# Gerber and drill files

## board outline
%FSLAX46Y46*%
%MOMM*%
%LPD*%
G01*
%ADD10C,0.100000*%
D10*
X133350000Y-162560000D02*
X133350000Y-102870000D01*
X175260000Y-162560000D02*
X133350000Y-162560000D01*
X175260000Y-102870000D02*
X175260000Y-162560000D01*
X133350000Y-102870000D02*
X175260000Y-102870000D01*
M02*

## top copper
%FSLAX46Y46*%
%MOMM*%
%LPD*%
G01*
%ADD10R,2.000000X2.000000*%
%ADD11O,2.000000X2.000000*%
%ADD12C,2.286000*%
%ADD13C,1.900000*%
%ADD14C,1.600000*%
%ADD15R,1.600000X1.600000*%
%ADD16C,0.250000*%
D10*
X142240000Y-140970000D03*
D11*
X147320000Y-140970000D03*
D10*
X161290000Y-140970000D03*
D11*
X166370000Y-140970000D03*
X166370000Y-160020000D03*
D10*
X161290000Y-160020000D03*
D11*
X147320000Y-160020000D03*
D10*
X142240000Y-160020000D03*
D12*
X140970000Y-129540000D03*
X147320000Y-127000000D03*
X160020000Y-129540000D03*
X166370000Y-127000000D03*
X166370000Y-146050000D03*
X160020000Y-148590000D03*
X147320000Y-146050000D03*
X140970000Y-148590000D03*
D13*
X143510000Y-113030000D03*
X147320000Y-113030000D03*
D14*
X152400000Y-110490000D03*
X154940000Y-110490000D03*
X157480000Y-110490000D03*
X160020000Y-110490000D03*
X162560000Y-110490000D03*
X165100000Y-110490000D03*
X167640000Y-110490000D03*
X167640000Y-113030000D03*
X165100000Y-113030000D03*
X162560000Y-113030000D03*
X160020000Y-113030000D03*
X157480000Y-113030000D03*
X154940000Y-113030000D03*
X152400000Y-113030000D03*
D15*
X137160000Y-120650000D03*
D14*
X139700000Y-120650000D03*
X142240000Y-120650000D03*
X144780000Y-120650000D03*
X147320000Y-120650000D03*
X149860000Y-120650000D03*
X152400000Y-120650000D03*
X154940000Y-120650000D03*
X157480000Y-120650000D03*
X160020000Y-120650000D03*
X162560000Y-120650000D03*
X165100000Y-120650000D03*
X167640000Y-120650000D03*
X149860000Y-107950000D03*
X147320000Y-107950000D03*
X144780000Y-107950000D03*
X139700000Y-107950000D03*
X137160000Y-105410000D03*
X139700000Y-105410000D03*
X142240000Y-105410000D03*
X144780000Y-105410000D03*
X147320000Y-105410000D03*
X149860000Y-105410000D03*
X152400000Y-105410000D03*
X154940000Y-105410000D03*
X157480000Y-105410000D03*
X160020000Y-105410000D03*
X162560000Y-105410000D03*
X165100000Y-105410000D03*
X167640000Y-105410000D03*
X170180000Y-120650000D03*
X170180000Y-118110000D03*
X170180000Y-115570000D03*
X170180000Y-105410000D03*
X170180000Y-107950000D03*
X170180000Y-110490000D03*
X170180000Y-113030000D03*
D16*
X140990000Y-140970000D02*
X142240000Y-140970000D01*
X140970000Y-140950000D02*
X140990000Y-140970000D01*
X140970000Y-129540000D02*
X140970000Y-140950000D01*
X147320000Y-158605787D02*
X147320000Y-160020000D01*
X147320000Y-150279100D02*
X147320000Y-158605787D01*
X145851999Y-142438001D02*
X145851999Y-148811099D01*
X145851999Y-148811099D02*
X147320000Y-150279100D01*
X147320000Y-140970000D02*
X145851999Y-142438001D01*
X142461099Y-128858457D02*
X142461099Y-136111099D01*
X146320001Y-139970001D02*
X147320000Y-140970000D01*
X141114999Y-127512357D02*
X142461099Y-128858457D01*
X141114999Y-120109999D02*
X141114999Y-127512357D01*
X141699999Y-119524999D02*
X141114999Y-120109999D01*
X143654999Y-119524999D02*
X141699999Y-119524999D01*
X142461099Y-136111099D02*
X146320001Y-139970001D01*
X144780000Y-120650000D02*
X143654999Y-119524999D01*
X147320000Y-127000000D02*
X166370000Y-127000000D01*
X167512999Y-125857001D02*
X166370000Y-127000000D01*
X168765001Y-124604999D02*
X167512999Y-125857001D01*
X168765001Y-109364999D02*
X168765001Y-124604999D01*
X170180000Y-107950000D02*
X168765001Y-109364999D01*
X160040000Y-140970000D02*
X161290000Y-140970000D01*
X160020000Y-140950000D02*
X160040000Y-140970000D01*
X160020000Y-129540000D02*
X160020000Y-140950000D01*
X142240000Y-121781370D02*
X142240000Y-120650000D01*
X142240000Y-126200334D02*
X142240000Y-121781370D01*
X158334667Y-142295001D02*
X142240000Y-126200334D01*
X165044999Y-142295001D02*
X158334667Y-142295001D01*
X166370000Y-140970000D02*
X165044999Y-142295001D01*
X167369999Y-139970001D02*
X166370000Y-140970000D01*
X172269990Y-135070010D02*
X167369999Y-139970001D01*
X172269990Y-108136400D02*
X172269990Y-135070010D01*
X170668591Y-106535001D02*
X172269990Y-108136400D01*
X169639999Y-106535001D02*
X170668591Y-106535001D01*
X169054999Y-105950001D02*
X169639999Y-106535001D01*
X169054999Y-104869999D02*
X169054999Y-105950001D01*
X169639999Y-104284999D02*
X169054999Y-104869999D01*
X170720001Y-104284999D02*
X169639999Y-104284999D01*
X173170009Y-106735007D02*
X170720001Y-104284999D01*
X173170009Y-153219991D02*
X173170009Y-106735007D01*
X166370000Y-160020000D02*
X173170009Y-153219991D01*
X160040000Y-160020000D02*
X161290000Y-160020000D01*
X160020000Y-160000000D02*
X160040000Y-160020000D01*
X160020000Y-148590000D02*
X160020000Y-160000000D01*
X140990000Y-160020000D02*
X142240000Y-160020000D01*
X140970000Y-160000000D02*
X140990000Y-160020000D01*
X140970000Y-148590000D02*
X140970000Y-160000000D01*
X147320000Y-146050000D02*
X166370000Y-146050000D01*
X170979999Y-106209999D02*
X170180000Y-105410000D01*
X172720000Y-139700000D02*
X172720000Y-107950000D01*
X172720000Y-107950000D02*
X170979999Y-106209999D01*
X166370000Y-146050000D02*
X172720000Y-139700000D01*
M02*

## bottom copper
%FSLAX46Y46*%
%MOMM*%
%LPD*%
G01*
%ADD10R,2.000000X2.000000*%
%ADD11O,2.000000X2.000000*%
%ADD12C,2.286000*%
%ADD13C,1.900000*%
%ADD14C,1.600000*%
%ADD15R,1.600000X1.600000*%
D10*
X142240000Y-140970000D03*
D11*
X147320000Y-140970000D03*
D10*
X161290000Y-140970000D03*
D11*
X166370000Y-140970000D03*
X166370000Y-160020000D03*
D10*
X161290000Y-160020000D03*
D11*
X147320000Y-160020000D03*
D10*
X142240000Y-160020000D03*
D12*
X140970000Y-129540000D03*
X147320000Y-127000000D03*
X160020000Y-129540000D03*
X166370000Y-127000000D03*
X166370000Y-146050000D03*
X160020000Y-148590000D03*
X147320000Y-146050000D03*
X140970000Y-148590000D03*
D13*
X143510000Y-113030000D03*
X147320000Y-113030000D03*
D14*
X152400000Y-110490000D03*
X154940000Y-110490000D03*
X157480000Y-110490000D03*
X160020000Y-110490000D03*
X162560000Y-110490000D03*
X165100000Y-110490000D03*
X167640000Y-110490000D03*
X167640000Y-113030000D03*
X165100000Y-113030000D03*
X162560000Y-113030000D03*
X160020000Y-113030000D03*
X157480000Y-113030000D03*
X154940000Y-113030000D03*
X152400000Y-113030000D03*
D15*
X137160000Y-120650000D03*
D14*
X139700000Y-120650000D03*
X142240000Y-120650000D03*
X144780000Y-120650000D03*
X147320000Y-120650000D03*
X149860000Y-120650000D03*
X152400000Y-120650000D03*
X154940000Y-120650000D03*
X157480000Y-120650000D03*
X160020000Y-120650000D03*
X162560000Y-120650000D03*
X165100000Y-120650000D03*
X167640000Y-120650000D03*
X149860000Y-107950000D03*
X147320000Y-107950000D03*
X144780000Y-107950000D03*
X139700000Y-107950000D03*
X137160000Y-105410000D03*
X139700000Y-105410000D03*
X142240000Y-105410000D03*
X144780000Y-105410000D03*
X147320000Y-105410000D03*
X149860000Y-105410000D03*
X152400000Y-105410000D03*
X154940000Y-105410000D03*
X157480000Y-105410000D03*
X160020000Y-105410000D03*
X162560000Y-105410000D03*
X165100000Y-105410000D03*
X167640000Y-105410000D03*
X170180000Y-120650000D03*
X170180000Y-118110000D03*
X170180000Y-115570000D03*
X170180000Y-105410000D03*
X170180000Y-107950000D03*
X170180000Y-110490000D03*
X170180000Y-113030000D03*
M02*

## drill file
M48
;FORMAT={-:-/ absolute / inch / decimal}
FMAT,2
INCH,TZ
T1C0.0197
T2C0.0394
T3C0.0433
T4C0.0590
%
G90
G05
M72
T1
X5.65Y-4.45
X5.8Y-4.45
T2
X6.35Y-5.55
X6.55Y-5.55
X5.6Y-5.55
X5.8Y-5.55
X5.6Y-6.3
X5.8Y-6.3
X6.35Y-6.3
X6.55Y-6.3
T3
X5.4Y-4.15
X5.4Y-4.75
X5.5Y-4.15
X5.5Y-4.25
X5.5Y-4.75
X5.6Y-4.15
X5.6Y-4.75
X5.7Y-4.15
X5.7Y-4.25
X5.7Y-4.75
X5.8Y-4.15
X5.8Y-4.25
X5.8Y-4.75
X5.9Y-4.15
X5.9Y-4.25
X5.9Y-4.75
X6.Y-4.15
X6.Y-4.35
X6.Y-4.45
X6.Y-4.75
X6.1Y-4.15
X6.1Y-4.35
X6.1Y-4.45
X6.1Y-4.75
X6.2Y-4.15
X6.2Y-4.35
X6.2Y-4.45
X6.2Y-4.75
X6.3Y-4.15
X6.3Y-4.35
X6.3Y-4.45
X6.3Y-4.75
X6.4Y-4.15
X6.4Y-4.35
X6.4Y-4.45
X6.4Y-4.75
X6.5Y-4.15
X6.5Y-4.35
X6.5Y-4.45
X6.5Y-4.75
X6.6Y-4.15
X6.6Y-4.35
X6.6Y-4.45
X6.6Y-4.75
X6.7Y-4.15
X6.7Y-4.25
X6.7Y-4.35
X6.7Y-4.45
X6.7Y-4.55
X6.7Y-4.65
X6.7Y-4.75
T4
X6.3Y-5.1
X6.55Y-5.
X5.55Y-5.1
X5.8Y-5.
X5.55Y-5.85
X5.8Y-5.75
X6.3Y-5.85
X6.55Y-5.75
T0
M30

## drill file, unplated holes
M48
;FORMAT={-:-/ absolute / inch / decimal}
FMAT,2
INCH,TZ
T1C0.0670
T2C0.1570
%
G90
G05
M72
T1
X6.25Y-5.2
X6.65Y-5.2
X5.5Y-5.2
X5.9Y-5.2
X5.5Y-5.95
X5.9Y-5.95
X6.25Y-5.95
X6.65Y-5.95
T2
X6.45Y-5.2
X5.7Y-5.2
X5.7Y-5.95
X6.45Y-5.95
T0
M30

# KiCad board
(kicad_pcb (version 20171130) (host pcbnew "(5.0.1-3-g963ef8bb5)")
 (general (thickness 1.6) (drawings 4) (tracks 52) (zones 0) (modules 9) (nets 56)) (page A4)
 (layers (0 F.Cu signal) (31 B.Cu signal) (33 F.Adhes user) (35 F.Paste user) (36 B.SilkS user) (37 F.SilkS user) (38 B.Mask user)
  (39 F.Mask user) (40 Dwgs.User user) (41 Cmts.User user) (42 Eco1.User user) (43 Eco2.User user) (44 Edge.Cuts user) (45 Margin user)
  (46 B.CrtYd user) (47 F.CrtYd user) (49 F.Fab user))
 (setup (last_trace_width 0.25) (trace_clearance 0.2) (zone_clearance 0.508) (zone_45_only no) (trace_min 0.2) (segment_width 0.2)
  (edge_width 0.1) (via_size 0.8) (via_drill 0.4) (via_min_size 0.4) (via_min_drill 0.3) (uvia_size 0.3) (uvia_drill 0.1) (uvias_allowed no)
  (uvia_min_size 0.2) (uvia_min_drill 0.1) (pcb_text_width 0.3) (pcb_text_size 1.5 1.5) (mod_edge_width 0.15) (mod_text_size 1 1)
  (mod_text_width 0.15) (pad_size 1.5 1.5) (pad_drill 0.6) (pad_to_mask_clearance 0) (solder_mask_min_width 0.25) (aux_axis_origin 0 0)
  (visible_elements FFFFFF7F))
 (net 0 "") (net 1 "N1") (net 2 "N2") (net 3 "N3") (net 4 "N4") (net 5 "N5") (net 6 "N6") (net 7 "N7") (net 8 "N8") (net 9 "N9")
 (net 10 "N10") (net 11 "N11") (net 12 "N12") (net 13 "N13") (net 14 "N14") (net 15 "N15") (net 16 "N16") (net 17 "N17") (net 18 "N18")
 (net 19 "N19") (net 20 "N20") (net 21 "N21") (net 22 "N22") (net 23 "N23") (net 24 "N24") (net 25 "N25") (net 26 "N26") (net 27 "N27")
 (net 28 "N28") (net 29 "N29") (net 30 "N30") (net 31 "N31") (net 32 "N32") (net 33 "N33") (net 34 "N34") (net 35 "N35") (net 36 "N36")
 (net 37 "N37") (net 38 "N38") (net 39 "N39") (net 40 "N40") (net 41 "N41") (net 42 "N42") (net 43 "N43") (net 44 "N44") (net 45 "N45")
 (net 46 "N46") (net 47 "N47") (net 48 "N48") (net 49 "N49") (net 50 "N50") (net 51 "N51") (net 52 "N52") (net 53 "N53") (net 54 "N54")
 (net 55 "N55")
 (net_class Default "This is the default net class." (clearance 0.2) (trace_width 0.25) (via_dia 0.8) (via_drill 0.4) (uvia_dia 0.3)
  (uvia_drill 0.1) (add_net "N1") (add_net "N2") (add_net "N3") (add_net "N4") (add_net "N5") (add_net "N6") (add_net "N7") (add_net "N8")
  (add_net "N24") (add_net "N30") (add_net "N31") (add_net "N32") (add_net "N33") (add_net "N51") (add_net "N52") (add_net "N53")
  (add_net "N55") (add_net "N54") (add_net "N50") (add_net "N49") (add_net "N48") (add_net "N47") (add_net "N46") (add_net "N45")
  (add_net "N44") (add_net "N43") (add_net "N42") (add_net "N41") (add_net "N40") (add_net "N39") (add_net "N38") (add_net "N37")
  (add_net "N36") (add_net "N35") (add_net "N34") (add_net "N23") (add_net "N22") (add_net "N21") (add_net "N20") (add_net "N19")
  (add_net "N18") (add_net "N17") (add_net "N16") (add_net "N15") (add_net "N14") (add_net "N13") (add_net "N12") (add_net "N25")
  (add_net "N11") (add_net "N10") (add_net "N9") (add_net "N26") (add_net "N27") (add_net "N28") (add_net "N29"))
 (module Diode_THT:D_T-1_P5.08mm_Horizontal (layer F.Cu) (at 142.24 140.97)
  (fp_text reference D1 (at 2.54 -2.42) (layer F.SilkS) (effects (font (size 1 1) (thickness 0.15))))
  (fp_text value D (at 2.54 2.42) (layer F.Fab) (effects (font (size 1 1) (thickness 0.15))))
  (pad 1 thru_hole rect (at 0 0) (size 2 2) (drill 1) (layers *.Cu *.Mask) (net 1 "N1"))
  (pad 2 thru_hole oval (at 5.08 0) (size 2 2) (drill 1) (layers *.Cu *.Mask) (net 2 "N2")))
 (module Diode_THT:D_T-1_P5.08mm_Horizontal (layer F.Cu) (at 161.29 140.97)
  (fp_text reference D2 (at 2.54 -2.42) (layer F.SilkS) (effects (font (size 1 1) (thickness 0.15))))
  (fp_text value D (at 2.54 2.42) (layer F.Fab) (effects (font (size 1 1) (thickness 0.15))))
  (pad 1 thru_hole rect (at 0 0) (size 2 2) (drill 1) (layers *.Cu *.Mask) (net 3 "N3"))
  (pad 2 thru_hole oval (at 5.08 0) (size 2 2) (drill 1) (layers *.Cu *.Mask) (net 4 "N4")))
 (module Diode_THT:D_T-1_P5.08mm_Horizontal (layer F.Cu) (at 161.29 160.02)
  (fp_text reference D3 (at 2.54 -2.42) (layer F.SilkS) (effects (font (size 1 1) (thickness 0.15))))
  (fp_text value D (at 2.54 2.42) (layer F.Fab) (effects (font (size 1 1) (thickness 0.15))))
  (pad 2 thru_hole oval (at 5.08 0) (size 2 2) (drill 1) (layers *.Cu *.Mask) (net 4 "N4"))
  (pad 1 thru_hole rect (at 0 0) (size 2 2) (drill 1) (layers *.Cu *.Mask) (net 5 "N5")))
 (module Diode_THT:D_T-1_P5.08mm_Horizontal (layer F.Cu) (at 142.24 160.02)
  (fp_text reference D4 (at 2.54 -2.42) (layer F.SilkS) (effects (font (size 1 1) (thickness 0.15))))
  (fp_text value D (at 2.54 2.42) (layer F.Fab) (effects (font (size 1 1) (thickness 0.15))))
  (pad 2 thru_hole oval (at 5.08 0) (size 2 2) (drill 1) (layers *.Cu *.Mask) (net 2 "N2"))
  (pad 1 thru_hole rect (at 0 0) (size 2 2) (drill 1) (layers *.Cu *.Mask) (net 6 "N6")))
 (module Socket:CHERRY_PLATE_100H (layer F.Cu) (at 144.78 132.08)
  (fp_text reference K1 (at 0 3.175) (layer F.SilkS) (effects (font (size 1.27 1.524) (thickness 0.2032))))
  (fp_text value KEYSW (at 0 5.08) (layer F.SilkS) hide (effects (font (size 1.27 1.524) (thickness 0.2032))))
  (pad HOLE np_thru_hole circle (at 5.08 0) (size 1.7018 1.7018) (drill 1.7018) (layers *.Cu))
  (pad HOLE np_thru_hole circle (at -5.08 0) (size 1.7018 1.7018) (drill 1.7018) (layers *.Cu))
  (pad HOLE np_thru_hole circle (at 0 0) (size 3.9878 3.9878) (drill 3.9878) (layers *.Cu))
  (pad 2 thru_hole circle (at -3.81 -2.54) (size 2.286 2.286) (drill 1.4986) (layers *.Cu *.SilkS *.Mask) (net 1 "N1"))
  (pad 1 thru_hole circle (at 2.54 -5.08) (size 2.286 2.286) (drill 1.4986) (layers *.Cu *.SilkS *.Mask) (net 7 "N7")))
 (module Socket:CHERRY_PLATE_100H (layer F.Cu) (at 163.83 132.08)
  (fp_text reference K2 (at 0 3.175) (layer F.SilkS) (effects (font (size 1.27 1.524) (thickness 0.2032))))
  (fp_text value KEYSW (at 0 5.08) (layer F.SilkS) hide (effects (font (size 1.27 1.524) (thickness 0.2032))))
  (pad HOLE np_thru_hole circle (at 5.08 0) (size 1.7018 1.7018) (drill 1.7018) (layers *.Cu))
  (pad HOLE np_thru_hole circle (at -5.08 0) (size 1.7018 1.7018) (drill 1.7018) (layers *.Cu))
  (pad HOLE np_thru_hole circle (at 0 0) (size 3.9878 3.9878) (drill 3.9878) (layers *.Cu))
  (pad 2 thru_hole circle (at -3.81 -2.54) (size 2.286 2.286) (drill 1.4986) (layers *.Cu *.SilkS *.Mask) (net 3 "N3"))
  (pad 1 thru_hole circle (at 2.54 -5.08) (size 2.286 2.286) (drill 1.4986) (layers *.Cu *.SilkS *.Mask) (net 7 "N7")))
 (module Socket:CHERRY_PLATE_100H (layer F.Cu) (at 163.83 151.13)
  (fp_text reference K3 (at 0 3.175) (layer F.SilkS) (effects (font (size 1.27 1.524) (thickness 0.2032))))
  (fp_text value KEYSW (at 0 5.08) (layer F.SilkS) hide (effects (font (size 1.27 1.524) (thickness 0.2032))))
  (pad 1 thru_hole circle (at 2.54 -5.08) (size 2.286 2.286) (drill 1.4986) (layers *.Cu *.SilkS *.Mask) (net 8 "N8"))
  (pad 2 thru_hole circle (at -3.81 -2.54) (size 2.286 2.286) (drill 1.4986) (layers *.Cu *.SilkS *.Mask) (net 5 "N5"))
  (pad HOLE np_thru_hole circle (at 0 0) (size 3.9878 3.9878) (drill 3.9878) (layers *.Cu))
  (pad HOLE np_thru_hole circle (at -5.08 0) (size 1.7018 1.7018) (drill 1.7018) (layers *.Cu))
  (pad HOLE np_thru_hole circle (at 5.08 0) (size 1.7018 1.7018) (drill 1.7018) (layers *.Cu)))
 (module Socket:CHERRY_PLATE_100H (layer F.Cu) (at 144.78 151.13)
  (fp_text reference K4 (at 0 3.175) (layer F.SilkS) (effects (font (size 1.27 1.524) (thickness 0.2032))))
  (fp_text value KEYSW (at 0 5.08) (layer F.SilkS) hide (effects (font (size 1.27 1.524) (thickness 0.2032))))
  (pad 1 thru_hole circle (at 2.54 -5.08) (size 2.286 2.286) (drill 1.4986) (layers *.Cu *.SilkS *.Mask) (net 8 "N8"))
  (pad 2 thru_hole circle (at -3.81 -2.54) (size 2.286 2.286) (drill 1.4986) (layers *.Cu *.SilkS *.Mask) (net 6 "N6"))
  (pad HOLE np_thru_hole circle (at 0 0) (size 3.9878 3.9878) (drill 3.9878) (layers *.Cu))
  (pad HOLE np_thru_hole circle (at -5.08 0) (size 1.7018 1.7018) (drill 1.7018) (layers *.Cu))
  (pad HOLE np_thru_hole circle (at 5.08 0) (size 1.7018 1.7018) (drill 1.7018) (layers *.Cu)))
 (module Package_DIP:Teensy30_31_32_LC (layer F.Cu) (at 153.67 113.03)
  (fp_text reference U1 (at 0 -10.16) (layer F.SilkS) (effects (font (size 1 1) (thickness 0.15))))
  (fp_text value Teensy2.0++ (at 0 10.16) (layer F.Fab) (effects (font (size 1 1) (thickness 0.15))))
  (pad 52 thru_hole circle (at -10.16 0) (size 1.9 1.9) (drill 0.5) (layers *.Cu *.Mask F.SilkS) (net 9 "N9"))
  (pad 52 thru_hole circle (at -6.35 0) (size 1.9 1.9) (drill 0.5) (layers *.Cu *.Mask F.SilkS) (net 9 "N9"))
  (pad 51 thru_hole circle (at -1.27 -2.54) (size 1.6 1.6) (drill 1.1) (layers *.Cu *.Mask) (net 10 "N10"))
  (pad 50 thru_hole circle (at 1.27 -2.54) (size 1.6 1.6) (drill 1.1) (layers *.Cu *.Mask) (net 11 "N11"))
  (pad 49 thru_hole circle (at 3.81 -2.54) (size 1.6 1.6) (drill 1.1) (layers *.Cu *.Mask) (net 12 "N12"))
  (pad 48 thru_hole circle (at 6.35 -2.54) (size 1.6 1.6) (drill 1.1) (layers *.Cu *.Mask) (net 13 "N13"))
  (pad 47 thru_hole circle (at 8.89 -2.54) (size 1.6 1.6) (drill 1.1) (layers *.Cu *.Mask) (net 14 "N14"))
  (pad 46 thru_hole circle (at 11.43 -2.54) (size 1.6 1.6) (drill 1.1) (layers *.Cu *.Mask) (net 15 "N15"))
  (pad 45 thru_hole circle (at 13.97 -2.54) (size 1.6 1.6) (drill 1.1) (layers *.Cu *.Mask) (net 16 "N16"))
  (pad 44 thru_hole circle (at 13.97 0) (size 1.6 1.6) (drill 1.1) (layers *.Cu *.Mask) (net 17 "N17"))
  (pad 43 thru_hole circle (at 11.43 0) (size 1.6 1.6) (drill 1.1) (layers *.Cu *.Mask) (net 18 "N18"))
  (pad 42 thru_hole circle (at 8.89 0) (size 1.6 1.6) (drill 1.1) (layers *.Cu *.Mask) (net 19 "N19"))
  (pad 41 thru_hole circle (at 6.35 0) (size 1.6 1.6) (drill 1.1) (layers *.Cu *.Mask) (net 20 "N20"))
  (pad 40 thru_hole circle (at 3.81 0) (size 1.6 1.6) (drill 1.1) (layers *.Cu *.Mask) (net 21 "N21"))
  (pad 39 thru_hole circle (at 1.27 0) (size 1.6 1.6) (drill 1.1) (layers *.Cu *.Mask) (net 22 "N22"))
  (pad 38 thru_hole circle (at -1.27 0) (size 1.6 1.6) (drill 1.1) (layers *.Cu *.Mask) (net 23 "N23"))
  (pad 1 thru_hole rect (at -16.51 7.62) (size 1.6 1.6) (drill 1.1) (layers *.Cu *.Mask F.SilkS) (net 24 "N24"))
  (pad 2 thru_hole circle (at -13.97 7.62) (size 1.6 1.6) (drill 1.1) (layers *.Cu *.Mask F.SilkS))
  (pad 3 thru_hole circle (at -11.43 7.62) (size 1.6 1.6) (drill 1.1) (layers *.Cu *.Mask F.SilkS) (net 4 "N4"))
  (pad 4 thru_hole circle (at -8.89 7.62) (size 1.6 1.6) (drill 1.1) (layers *.Cu *.Mask F.SilkS) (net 2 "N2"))
  (pad 5 thru_hole circle (at -6.35 7.62) (size 1.6 1.6) (drill 1.1) (layers *.Cu *.Mask F.SilkS) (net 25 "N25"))
  (pad 6 thru_hole circle (at -3.81 7.62) (size 1.6 1.6) (drill 1.1) (layers *.Cu *.Mask F.SilkS) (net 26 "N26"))
  (pad 7 thru_hole circle (at -1.27 7.62) (size 1.6 1.6) (drill 1.1) (layers *.Cu *.Mask F.SilkS) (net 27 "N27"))
  (pad 8 thru_hole circle (at 1.27 7.62) (size 1.6 1.6) (drill 1.1) (layers *.Cu *.Mask F.SilkS) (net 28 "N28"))
  (pad 9 thru_hole circle (at 3.81 7.62) (size 1.6 1.6) (drill 1.1) (layers *.Cu *.Mask F.SilkS) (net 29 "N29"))
  (pad 10 thru_hole circle (at 6.35 7.62) (size 1.6 1.6) (drill 1.1) (layers *.Cu *.Mask F.SilkS) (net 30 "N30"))
  (pad 11 thru_hole circle (at 8.89 7.62) (size 1.6 1.6) (drill 1.1) (layers *.Cu *.Mask F.SilkS) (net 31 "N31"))
  (pad 12 thru_hole circle (at 11.43 7.62) (size 1.6 1.6) (drill 1.1) (layers *.Cu *.Mask F.SilkS) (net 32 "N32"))
  (pad 13 thru_hole circle (at 13.97 7.62) (size 1.6 1.6) (drill 1.1) (layers *.Cu *.Mask F.SilkS) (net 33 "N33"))
  (pad 37 thru_hole circle (at -3.81 -5.08) (size 1.6 1.6) (drill 1.1) (layers *.Cu *.Mask F.SilkS) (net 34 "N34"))
  (pad 36 thru_hole circle (at -6.35 -5.08) (size 1.6 1.6) (drill 1.1) (layers *.Cu *.Mask F.SilkS) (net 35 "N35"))
  (pad 35 thru_hole circle (at -8.89 -5.08) (size 1.6 1.6) (drill 1.1) (layers *.Cu *.Mask F.SilkS) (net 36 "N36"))
  (pad 34 thru_hole circle (at -13.97 -5.08) (size 1.6 1.6) (drill 1.1) (layers *.Cu *.Mask F.SilkS) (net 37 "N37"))
  (pad 33 thru_hole circle (at -16.51 -7.62) (size 1.6 1.6) (drill 1.1) (layers *.Cu *.Mask F.SilkS) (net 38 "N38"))
  (pad 32 thru_hole circle (at -13.97 -7.62) (size 1.6 1.6) (drill 1.1) (layers *.Cu *.Mask F.SilkS) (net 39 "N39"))
  (pad 31 thru_hole circle (at -11.43 -7.62) (size 1.6 1.6) (drill 1.1) (layers *.Cu *.Mask F.SilkS) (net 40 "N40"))
  (pad 30 thru_hole circle (at -8.89 -7.62) (size 1.6 1.6) (drill 1.1) (layers *.Cu *.Mask F.SilkS) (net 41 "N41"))
  (pad 29 thru_hole circle (at -6.35 -7.62) (size 1.6 1.6) (drill 1.1) (layers *.Cu *.Mask F.SilkS) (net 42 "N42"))
  (pad 28 thru_hole circle (at -3.81 -7.62) (size 1.6 1.6) (drill 1.1) (layers *.Cu *.Mask F.SilkS) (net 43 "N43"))
  (pad 27 thru_hole circle (at -1.27 -7.62) (size 1.6 1.6) (drill 1.1) (layers *.Cu *.Mask F.SilkS) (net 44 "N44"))
  (pad 26 thru_hole circle (at 1.27 -7.62) (size 1.6 1.6) (drill 1.1) (layers *.Cu *.Mask F.SilkS) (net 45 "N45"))
  (pad 25 thru_hole circle (at 3.81 -7.62) (size 1.6 1.6) (drill 1.1) (layers *.Cu *.Mask F.SilkS) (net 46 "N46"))
  (pad 24 thru_hole circle (at 6.35 -7.62) (size 1.6 1.6) (drill 1.1) (layers *.Cu *.Mask F.SilkS) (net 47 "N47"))
  (pad 23 thru_hole circle (at 8.89 -7.62) (size 1.6 1.6) (drill 1.1) (layers *.Cu *.Mask F.SilkS) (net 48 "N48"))
  (pad 22 thru_hole circle (at 11.43 -7.62) (size 1.6 1.6) (drill 1.1) (layers *.Cu *.Mask F.SilkS) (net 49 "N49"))
  (pad 21 thru_hole circle (at 13.97 -7.62) (size 1.6 1.6) (drill 1.1) (layers *.Cu *.Mask F.SilkS) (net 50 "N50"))
  (pad 14 thru_hole circle (at 16.51 7.62) (size 1.6 1.6) (drill 1.1) (layers *.Cu *.Mask F.SilkS) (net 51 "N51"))
  (pad 15 thru_hole circle (at 16.51 5.08) (size 1.6 1.6) (drill 1.1) (layers *.Cu *.Mask F.SilkS) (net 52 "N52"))
  (pad 16 thru_hole circle (at 16.51 2.54) (size 1.6 1.6) (drill 1.1) (layers *.Cu *.Mask F.SilkS) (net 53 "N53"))
  (pad 20 thru_hole circle (at 16.51 -7.62) (size 1.6 1.6) (drill 1.1) (layers *.Cu *.Mask F.SilkS) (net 8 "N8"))
  (pad 19 thru_hole circle (at 16.51 -5.08) (size 1.6 1.6) (drill 1.1) (layers *.Cu *.Mask F.SilkS) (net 7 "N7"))
  (pad 18 thru_hole circle (at 16.51 -2.54) (size 1.6 1.6) (drill 1.1) (layers *.Cu *.Mask F.SilkS) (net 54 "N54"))
  (pad 17 thru_hole circle (at 16.51 0) (size 1.6 1.6) (drill 1.1) (layers *.Cu *.Mask F.SilkS) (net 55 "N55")))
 (gr_line (start 133.35 162.56) (end 133.35 102.87) (layer Edge.Cuts) (width 0.1))
 (gr_line (start 175.26 162.56) (end 133.35 162.56) (layer Edge.Cuts) (width 0.1))
 (gr_line (start 175.26 102.87) (end 175.26 162.56) (layer Edge.Cuts) (width 0.1))
 (gr_line (start 133.35 102.87) (end 175.26 102.87) (layer Edge.Cuts) (width 0.1))
 (segment (start 140.99 140.97) (end 142.24 140.97) (width 0.25) (layer F.Cu) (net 1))
 (segment (start 140.97 140.95) (end 140.99 140.97) (width 0.25) (layer F.Cu) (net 1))
 (segment (start 140.97 129.54) (end 140.97 140.95) (width 0.25) (layer F.Cu) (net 1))
 (segment (start 147.32 158.605787) (end 147.32 160.02) (width 0.25) (layer F.Cu) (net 2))
 (segment (start 147.32 150.2791) (end 147.32 158.605787) (width 0.25) (layer F.Cu) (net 2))
 (segment (start 145.851999 142.438001) (end 145.851999 148.811099) (width 0.25) (layer F.Cu) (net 2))
 (segment (start 145.851999 148.811099) (end 147.32 150.2791) (width 0.25) (layer F.Cu) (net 2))
 (segment (start 147.32 140.97) (end 145.851999 142.438001) (width 0.25) (layer F.Cu) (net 2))
 (segment (start 142.461099 128.858457) (end 142.461099 136.111099) (width 0.25) (layer F.Cu) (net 2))
 (segment (start 146.320001 139.970001) (end 147.32 140.97) (width 0.25) (layer F.Cu) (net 2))
 (segment (start 141.114999 127.512357) (end 142.461099 128.858457) (width 0.25) (layer F.Cu) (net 2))
 (segment (start 141.114999 120.109999) (end 141.114999 127.512357) (width 0.25) (layer F.Cu) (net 2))
 (segment (start 141.699999 119.524999) (end 141.114999 120.109999) (width 0.25) (layer F.Cu) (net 2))
 (segment (start 143.654999 119.524999) (end 141.699999 119.524999) (width 0.25) (layer F.Cu) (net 2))
 (segment (start 142.461099 136.111099) (end 146.320001 139.970001) (width 0.25) (layer F.Cu) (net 2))
 (segment (start 144.78 120.65) (end 143.654999 119.524999) (width 0.25) (layer F.Cu) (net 2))
 (segment (start 147.32 127) (end 166.37 127) (width 0.25) (layer F.Cu) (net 7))
 (segment (start 167.512999 125.857001) (end 166.37 127) (width 0.25) (layer F.Cu) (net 7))
 (segment (start 168.765001 124.604999) (end 167.512999 125.857001) (width 0.25) (layer F.Cu) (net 7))
 (segment (start 168.765001 109.364999) (end 168.765001 124.604999) (width 0.25) (layer F.Cu) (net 7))
 (segment (start 170.18 107.95) (end 168.765001 109.364999) (width 0.25) (layer F.Cu) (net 7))
 (segment (start 160.04 140.97) (end 161.29 140.97) (width 0.25) (layer F.Cu) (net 3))
 (segment (start 160.02 140.95) (end 160.04 140.97) (width 0.25) (layer F.Cu) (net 3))
 (segment (start 160.02 129.54) (end 160.02 140.95) (width 0.25) (layer F.Cu) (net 3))
 (segment (start 142.24 121.78137) (end 142.24 120.65) (width 0.25) (layer F.Cu) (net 4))
 (segment (start 142.24 126.200334) (end 142.24 121.78137) (width 0.25) (layer F.Cu) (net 4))
 (segment (start 158.334667 142.295001) (end 142.24 126.200334) (width 0.25) (layer F.Cu) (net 4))
 (segment (start 165.044999 142.295001) (end 158.334667 142.295001) (width 0.25) (layer F.Cu) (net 4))
 (segment (start 166.37 140.97) (end 165.044999 142.295001) (width 0.25) (layer F.Cu) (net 4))
 (segment (start 167.369999 139.970001) (end 166.37 140.97) (width 0.25) (layer F.Cu) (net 4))
 (segment (start 172.26999 135.07001) (end 167.369999 139.970001) (width 0.25) (layer F.Cu) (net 4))
 (segment (start 172.26999 108.1364) (end 172.26999 135.07001) (width 0.25) (layer F.Cu) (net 4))
 (segment (start 170.668591 106.535001) (end 172.26999 108.1364) (width 0.25) (layer F.Cu) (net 4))
 (segment (start 169.639999 106.535001) (end 170.668591 106.535001) (width 0.25) (layer F.Cu) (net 4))
 (segment (start 169.054999 105.950001) (end 169.639999 106.535001) (width 0.25) (layer F.Cu) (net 4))
 (segment (start 169.054999 104.869999) (end 169.054999 105.950001) (width 0.25) (layer F.Cu) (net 4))
 (segment (start 169.639999 104.284999) (end 169.054999 104.869999) (width 0.25) (layer F.Cu) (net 4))
 (segment (start 170.720001 104.284999) (end 169.639999 104.284999) (width 0.25) (layer F.Cu) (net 4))
 (segment (start 173.170009 106.735007) (end 170.720001 104.284999) (width 0.25) (layer F.Cu) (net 4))
 (segment (start 173.170009 153.219991) (end 173.170009 106.735007) (width 0.25) (layer F.Cu) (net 4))
 (segment (start 166.37 160.02) (end 173.170009 153.219991) (width 0.25) (layer F.Cu) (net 4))
 (segment (start 160.04 160.02) (end 161.29 160.02) (width 0.25) (layer F.Cu) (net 5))
 (segment (start 160.02 160) (end 160.04 160.02) (width 0.25) (layer F.Cu) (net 5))
 (segment (start 160.02 148.59) (end 160.02 160) (width 0.25) (layer F.Cu) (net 5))
 (segment (start 140.99 160.02) (end 142.24 160.02) (width 0.25) (layer F.Cu) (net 6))
 (segment (start 140.97 160) (end 140.99 160.02) (width 0.25) (layer F.Cu) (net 6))
 (segment (start 140.97 148.59) (end 140.97 160) (width 0.25) (layer F.Cu) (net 6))
 (segment (start 147.32 146.05) (end 166.37 146.05) (width 0.25) (layer F.Cu) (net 8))
 (segment (start 170.979999 106.209999) (end 170.18 105.41) (width 0.25) (layer F.Cu) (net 8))
 (segment (start 172.72 139.7) (end 172.72 107.95) (width 0.25) (layer F.Cu) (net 8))
 (segment (start 172.72 107.95) (end 170.979999 106.209999) (width 0.25) (layer F.Cu) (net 8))
 (segment (start 166.37 146.05) (end 172.72 139.7) (width 0.25) (layer F.Cu) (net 8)))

